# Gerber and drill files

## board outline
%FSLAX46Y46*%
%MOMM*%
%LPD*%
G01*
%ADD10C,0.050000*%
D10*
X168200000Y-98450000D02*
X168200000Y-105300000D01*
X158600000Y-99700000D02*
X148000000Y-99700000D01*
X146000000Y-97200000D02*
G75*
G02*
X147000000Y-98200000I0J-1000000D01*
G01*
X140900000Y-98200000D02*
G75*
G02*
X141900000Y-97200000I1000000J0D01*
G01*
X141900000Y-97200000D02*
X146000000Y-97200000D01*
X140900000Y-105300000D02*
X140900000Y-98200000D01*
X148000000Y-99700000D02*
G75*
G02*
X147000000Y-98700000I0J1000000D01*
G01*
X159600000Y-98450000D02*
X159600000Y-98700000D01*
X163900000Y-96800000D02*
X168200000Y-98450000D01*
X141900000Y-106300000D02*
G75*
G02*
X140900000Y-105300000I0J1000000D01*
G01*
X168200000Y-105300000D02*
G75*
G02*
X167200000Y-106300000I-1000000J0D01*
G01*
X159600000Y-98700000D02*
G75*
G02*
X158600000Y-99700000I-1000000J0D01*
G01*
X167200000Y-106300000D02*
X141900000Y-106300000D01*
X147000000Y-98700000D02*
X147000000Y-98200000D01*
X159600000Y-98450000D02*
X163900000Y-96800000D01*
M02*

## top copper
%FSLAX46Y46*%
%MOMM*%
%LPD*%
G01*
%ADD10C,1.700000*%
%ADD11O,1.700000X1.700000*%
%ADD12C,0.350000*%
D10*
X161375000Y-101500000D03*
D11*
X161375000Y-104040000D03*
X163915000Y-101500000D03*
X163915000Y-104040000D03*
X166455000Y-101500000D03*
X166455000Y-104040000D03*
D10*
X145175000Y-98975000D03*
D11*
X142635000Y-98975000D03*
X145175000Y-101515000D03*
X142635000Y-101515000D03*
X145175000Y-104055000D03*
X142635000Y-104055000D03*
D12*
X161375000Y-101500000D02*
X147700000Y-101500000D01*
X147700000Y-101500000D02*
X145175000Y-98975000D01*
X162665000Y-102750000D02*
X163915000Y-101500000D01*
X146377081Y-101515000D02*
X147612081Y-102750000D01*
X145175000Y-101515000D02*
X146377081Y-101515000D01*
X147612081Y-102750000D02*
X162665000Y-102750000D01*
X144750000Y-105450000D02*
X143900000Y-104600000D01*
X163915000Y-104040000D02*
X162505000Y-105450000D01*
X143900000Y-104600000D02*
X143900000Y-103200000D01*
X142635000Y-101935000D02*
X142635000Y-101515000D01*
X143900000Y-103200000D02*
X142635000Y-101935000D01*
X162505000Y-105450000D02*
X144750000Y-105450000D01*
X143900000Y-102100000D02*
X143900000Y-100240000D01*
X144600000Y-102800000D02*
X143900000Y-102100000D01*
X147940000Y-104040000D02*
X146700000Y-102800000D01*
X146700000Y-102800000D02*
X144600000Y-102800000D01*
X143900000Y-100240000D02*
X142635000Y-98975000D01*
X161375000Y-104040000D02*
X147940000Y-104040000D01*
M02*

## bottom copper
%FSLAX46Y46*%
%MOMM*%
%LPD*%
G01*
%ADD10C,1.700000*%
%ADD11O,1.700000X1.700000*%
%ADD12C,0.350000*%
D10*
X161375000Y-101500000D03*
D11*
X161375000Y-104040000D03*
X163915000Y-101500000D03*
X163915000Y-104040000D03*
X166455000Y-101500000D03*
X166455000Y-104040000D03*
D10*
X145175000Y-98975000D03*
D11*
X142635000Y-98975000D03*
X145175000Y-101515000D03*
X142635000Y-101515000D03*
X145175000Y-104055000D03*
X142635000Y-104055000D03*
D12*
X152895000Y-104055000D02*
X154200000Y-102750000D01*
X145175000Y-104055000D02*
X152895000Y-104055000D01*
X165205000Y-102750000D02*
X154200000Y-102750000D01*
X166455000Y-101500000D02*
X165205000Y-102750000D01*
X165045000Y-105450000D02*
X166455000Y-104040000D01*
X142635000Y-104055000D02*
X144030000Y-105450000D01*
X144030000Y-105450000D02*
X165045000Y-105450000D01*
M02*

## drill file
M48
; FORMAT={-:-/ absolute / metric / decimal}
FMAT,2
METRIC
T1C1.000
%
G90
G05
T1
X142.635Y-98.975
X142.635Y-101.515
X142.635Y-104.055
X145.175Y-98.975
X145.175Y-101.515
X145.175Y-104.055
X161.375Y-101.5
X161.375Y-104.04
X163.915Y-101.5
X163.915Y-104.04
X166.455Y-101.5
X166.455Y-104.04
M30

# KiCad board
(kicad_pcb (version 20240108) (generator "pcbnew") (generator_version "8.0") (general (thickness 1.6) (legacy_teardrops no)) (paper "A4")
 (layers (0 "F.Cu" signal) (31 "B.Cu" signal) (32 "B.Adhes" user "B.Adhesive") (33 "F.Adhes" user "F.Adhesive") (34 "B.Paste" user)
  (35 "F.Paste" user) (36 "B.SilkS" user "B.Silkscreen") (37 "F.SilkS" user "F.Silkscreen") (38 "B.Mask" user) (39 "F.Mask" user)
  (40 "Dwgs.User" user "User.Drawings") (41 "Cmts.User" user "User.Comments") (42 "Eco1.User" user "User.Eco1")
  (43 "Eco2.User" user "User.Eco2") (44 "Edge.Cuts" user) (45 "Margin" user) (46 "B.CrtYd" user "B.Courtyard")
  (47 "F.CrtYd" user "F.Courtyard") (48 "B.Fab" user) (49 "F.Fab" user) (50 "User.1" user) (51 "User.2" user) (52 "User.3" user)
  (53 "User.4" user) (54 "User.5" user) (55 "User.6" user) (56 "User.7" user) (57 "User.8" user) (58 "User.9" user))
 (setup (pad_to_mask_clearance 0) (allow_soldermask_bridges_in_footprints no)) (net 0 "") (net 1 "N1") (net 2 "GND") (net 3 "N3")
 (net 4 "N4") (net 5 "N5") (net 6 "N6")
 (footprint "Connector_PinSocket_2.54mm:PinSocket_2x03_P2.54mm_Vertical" (layer "F.Cu") (at 161.375 101.5 90)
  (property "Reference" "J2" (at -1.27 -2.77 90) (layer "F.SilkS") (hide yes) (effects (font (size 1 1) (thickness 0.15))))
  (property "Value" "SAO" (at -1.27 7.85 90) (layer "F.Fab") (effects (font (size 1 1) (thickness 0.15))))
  (pad "1" thru_hole circle (at 0 0 90) (size 1.7 1.7) (drill 1) (layers "*.Cu" "*.Mask") (remove_unused_layers no) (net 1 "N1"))
  (pad "2" thru_hole oval (at -2.54 0 90) (size 1.7 1.7) (drill 1) (layers "*.Cu" "*.Mask") (remove_unused_layers no) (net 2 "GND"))
  (pad "3" thru_hole oval (at 0 2.54 90) (size 1.7 1.7) (drill 1) (layers "*.Cu" "*.Mask") (remove_unused_layers no) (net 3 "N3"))
  (pad "4" thru_hole oval (at -2.54 2.54 90) (size 1.7 1.7) (drill 1) (layers "*.Cu" "*.Mask") (remove_unused_layers no) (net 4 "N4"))
  (pad "5" thru_hole oval (at 0 5.08 90) (size 1.7 1.7) (drill 1) (layers "*.Cu" "*.Mask") (remove_unused_layers no) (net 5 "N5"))
  (pad "6" thru_hole oval (at -2.54 5.08 90) (size 1.7 1.7) (drill 1) (layers "*.Cu" "*.Mask") (remove_unused_layers no) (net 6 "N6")))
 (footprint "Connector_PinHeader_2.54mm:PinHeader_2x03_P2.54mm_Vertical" (layer "B.Cu") (at 145.175 98.975 180)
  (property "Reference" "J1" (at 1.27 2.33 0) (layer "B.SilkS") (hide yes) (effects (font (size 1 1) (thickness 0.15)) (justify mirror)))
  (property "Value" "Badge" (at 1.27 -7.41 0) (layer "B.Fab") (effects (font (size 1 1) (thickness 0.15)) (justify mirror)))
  (pad "1" thru_hole circle (at 0 0 180) (size 1.7 1.7) (drill 1) (layers "*.Cu" "*.Mask") (remove_unused_layers no) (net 1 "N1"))
  (pad "2" thru_hole oval (at 2.54 0 180) (size 1.7 1.7) (drill 1) (layers "*.Cu" "*.Mask") (remove_unused_layers no) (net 2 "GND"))
  (pad "3" thru_hole oval (at 0 -2.54 180) (size 1.7 1.7) (drill 1) (layers "*.Cu" "*.Mask") (remove_unused_layers no) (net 3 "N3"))
  (pad "4" thru_hole oval (at 2.54 -2.54 180) (size 1.7 1.7) (drill 1) (layers "*.Cu" "*.Mask") (remove_unused_layers no) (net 4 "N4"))
  (pad "5" thru_hole oval (at 0 -5.08 180) (size 1.7 1.7) (drill 1) (layers "*.Cu" "*.Mask") (remove_unused_layers no) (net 5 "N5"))
  (pad "6" thru_hole oval (at 2.54 -5.08 180) (size 1.7 1.7) (drill 1) (layers "*.Cu" "*.Mask") (remove_unused_layers no) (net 6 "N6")))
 (gr_line (start 168.2 98.45) (end 168.2 105.3) (stroke (width 0.05) (type default)) (layer "Edge.Cuts"))
 (gr_line (start 158.6 99.7) (end 148 99.7) (stroke (width 0.05) (type default)) (layer "Edge.Cuts"))
 (gr_arc (start 146 97.2) (mid 146.707107 97.492893) (end 147 98.2) (stroke (width 0.05) (type default)) (layer "Edge.Cuts"))
 (gr_arc (start 140.9 98.2) (mid 141.192893 97.492893) (end 141.9 97.2) (stroke (width 0.05) (type default)) (layer "Edge.Cuts"))
 (gr_line (start 141.9 97.2) (end 146 97.2) (stroke (width 0.05) (type default)) (layer "Edge.Cuts"))
 (gr_line (start 140.9 105.3) (end 140.9 98.2) (stroke (width 0.05) (type default)) (layer "Edge.Cuts"))
 (gr_arc (start 148 99.7) (mid 147.292893 99.407107) (end 147 98.7) (stroke (width 0.05) (type default)) (layer "Edge.Cuts"))
 (gr_line (start 159.6 98.45) (end 159.6 98.7) (stroke (width 0.05) (type default)) (layer "Edge.Cuts"))
 (gr_line (start 163.9 96.8) (end 168.2 98.45) (stroke (width 0.05) (type default)) (layer "Edge.Cuts"))
 (gr_arc (start 141.9 106.3) (mid 141.192893 106.007107) (end 140.9 105.3) (stroke (width 0.05) (type default)) (layer "Edge.Cuts"))
 (gr_arc (start 168.2 105.3) (mid 167.907107 106.007107) (end 167.2 106.3) (stroke (width 0.05) (type default)) (layer "Edge.Cuts"))
 (gr_arc (start 159.6 98.7) (mid 159.307107 99.407107) (end 158.6 99.7) (stroke (width 0.05) (type default)) (layer "Edge.Cuts"))
 (gr_line (start 167.2 106.3) (end 141.9 106.3) (stroke (width 0.05) (type default)) (layer "Edge.Cuts"))
 (gr_line (start 147 98.7) (end 147 98.2) (stroke (width 0.05) (type default)) (layer "Edge.Cuts"))
 (gr_line (start 159.6 98.45) (end 163.9 96.8) (stroke (width 0.05) (type default)) (layer "Edge.Cuts"))
 (segment (start 152.895 104.055) (end 154.2 102.75) (width 0.35) (layer "B.Cu") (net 5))
 (segment (start 145.175 104.055) (end 152.895 104.055) (width 0.35) (layer "B.Cu") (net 5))
 (segment (start 165.205 102.75) (end 154.2 102.75) (width 0.35) (layer "B.Cu") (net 5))
 (segment (start 166.455 101.5) (end 165.205 102.75) (width 0.35) (layer "B.Cu") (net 5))
 (segment (start 161.375 101.5) (end 147.7 101.5) (width 0.35) (layer "F.Cu") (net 1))
 (segment (start 147.7 101.5) (end 145.175 98.975) (width 0.35) (layer "F.Cu") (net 1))
 (segment (start 162.665 102.75) (end 163.915 101.5) (width 0.35) (layer "F.Cu") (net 3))
 (segment (start 146.377081 101.515) (end 147.612081 102.75) (width 0.35) (layer "F.Cu") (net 3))
 (segment (start 145.175 101.515) (end 146.377081 101.515) (width 0.35) (layer "F.Cu") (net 3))
 (segment (start 147.612081 102.75) (end 162.665 102.75) (width 0.35) (layer "F.Cu") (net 3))
 (segment (start 165.045 105.45) (end 166.455 104.04) (width 0.35) (layer "B.Cu") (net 6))
 (segment (start 142.635 104.055) (end 144.03 105.45) (width 0.35) (layer "B.Cu") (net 6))
 (segment (start 144.03 105.45) (end 165.045 105.45) (width 0.35) (layer "B.Cu") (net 6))
 (segment (start 144.75 105.45) (end 143.9 104.6) (width 0.35) (layer "F.Cu") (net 4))
 (segment (start 163.915 104.04) (end 162.505 105.45) (width 0.35) (layer "F.Cu") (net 4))
 (segment (start 143.9 104.6) (end 143.9 103.2) (width 0.35) (layer "F.Cu") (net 4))
 (segment (start 142.635 101.935) (end 142.635 101.515) (width 0.35) (layer "F.Cu") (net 4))
 (segment (start 143.9 103.2) (end 142.635 101.935) (width 0.35) (layer "F.Cu") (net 4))
 (segment (start 162.505 105.45) (end 144.75 105.45) (width 0.35) (layer "F.Cu") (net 4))
 (segment (start 143.9 102.1) (end 143.9 100.24) (width 0.35) (layer "F.Cu") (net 2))
 (segment (start 144.6 102.8) (end 143.9 102.1) (width 0.35) (layer "F.Cu") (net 2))
 (segment (start 147.94 104.04) (end 146.7 102.8) (width 0.35) (layer "F.Cu") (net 2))
 (segment (start 146.7 102.8) (end 144.6 102.8) (width 0.35) (layer "F.Cu") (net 2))
 (segment (start 143.9 100.24) (end 142.635 98.975) (width 0.35) (layer "F.Cu") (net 2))
 (segment (start 161.375 104.04) (end 147.94 104.04) (width 0.35) (layer "F.Cu") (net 2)))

